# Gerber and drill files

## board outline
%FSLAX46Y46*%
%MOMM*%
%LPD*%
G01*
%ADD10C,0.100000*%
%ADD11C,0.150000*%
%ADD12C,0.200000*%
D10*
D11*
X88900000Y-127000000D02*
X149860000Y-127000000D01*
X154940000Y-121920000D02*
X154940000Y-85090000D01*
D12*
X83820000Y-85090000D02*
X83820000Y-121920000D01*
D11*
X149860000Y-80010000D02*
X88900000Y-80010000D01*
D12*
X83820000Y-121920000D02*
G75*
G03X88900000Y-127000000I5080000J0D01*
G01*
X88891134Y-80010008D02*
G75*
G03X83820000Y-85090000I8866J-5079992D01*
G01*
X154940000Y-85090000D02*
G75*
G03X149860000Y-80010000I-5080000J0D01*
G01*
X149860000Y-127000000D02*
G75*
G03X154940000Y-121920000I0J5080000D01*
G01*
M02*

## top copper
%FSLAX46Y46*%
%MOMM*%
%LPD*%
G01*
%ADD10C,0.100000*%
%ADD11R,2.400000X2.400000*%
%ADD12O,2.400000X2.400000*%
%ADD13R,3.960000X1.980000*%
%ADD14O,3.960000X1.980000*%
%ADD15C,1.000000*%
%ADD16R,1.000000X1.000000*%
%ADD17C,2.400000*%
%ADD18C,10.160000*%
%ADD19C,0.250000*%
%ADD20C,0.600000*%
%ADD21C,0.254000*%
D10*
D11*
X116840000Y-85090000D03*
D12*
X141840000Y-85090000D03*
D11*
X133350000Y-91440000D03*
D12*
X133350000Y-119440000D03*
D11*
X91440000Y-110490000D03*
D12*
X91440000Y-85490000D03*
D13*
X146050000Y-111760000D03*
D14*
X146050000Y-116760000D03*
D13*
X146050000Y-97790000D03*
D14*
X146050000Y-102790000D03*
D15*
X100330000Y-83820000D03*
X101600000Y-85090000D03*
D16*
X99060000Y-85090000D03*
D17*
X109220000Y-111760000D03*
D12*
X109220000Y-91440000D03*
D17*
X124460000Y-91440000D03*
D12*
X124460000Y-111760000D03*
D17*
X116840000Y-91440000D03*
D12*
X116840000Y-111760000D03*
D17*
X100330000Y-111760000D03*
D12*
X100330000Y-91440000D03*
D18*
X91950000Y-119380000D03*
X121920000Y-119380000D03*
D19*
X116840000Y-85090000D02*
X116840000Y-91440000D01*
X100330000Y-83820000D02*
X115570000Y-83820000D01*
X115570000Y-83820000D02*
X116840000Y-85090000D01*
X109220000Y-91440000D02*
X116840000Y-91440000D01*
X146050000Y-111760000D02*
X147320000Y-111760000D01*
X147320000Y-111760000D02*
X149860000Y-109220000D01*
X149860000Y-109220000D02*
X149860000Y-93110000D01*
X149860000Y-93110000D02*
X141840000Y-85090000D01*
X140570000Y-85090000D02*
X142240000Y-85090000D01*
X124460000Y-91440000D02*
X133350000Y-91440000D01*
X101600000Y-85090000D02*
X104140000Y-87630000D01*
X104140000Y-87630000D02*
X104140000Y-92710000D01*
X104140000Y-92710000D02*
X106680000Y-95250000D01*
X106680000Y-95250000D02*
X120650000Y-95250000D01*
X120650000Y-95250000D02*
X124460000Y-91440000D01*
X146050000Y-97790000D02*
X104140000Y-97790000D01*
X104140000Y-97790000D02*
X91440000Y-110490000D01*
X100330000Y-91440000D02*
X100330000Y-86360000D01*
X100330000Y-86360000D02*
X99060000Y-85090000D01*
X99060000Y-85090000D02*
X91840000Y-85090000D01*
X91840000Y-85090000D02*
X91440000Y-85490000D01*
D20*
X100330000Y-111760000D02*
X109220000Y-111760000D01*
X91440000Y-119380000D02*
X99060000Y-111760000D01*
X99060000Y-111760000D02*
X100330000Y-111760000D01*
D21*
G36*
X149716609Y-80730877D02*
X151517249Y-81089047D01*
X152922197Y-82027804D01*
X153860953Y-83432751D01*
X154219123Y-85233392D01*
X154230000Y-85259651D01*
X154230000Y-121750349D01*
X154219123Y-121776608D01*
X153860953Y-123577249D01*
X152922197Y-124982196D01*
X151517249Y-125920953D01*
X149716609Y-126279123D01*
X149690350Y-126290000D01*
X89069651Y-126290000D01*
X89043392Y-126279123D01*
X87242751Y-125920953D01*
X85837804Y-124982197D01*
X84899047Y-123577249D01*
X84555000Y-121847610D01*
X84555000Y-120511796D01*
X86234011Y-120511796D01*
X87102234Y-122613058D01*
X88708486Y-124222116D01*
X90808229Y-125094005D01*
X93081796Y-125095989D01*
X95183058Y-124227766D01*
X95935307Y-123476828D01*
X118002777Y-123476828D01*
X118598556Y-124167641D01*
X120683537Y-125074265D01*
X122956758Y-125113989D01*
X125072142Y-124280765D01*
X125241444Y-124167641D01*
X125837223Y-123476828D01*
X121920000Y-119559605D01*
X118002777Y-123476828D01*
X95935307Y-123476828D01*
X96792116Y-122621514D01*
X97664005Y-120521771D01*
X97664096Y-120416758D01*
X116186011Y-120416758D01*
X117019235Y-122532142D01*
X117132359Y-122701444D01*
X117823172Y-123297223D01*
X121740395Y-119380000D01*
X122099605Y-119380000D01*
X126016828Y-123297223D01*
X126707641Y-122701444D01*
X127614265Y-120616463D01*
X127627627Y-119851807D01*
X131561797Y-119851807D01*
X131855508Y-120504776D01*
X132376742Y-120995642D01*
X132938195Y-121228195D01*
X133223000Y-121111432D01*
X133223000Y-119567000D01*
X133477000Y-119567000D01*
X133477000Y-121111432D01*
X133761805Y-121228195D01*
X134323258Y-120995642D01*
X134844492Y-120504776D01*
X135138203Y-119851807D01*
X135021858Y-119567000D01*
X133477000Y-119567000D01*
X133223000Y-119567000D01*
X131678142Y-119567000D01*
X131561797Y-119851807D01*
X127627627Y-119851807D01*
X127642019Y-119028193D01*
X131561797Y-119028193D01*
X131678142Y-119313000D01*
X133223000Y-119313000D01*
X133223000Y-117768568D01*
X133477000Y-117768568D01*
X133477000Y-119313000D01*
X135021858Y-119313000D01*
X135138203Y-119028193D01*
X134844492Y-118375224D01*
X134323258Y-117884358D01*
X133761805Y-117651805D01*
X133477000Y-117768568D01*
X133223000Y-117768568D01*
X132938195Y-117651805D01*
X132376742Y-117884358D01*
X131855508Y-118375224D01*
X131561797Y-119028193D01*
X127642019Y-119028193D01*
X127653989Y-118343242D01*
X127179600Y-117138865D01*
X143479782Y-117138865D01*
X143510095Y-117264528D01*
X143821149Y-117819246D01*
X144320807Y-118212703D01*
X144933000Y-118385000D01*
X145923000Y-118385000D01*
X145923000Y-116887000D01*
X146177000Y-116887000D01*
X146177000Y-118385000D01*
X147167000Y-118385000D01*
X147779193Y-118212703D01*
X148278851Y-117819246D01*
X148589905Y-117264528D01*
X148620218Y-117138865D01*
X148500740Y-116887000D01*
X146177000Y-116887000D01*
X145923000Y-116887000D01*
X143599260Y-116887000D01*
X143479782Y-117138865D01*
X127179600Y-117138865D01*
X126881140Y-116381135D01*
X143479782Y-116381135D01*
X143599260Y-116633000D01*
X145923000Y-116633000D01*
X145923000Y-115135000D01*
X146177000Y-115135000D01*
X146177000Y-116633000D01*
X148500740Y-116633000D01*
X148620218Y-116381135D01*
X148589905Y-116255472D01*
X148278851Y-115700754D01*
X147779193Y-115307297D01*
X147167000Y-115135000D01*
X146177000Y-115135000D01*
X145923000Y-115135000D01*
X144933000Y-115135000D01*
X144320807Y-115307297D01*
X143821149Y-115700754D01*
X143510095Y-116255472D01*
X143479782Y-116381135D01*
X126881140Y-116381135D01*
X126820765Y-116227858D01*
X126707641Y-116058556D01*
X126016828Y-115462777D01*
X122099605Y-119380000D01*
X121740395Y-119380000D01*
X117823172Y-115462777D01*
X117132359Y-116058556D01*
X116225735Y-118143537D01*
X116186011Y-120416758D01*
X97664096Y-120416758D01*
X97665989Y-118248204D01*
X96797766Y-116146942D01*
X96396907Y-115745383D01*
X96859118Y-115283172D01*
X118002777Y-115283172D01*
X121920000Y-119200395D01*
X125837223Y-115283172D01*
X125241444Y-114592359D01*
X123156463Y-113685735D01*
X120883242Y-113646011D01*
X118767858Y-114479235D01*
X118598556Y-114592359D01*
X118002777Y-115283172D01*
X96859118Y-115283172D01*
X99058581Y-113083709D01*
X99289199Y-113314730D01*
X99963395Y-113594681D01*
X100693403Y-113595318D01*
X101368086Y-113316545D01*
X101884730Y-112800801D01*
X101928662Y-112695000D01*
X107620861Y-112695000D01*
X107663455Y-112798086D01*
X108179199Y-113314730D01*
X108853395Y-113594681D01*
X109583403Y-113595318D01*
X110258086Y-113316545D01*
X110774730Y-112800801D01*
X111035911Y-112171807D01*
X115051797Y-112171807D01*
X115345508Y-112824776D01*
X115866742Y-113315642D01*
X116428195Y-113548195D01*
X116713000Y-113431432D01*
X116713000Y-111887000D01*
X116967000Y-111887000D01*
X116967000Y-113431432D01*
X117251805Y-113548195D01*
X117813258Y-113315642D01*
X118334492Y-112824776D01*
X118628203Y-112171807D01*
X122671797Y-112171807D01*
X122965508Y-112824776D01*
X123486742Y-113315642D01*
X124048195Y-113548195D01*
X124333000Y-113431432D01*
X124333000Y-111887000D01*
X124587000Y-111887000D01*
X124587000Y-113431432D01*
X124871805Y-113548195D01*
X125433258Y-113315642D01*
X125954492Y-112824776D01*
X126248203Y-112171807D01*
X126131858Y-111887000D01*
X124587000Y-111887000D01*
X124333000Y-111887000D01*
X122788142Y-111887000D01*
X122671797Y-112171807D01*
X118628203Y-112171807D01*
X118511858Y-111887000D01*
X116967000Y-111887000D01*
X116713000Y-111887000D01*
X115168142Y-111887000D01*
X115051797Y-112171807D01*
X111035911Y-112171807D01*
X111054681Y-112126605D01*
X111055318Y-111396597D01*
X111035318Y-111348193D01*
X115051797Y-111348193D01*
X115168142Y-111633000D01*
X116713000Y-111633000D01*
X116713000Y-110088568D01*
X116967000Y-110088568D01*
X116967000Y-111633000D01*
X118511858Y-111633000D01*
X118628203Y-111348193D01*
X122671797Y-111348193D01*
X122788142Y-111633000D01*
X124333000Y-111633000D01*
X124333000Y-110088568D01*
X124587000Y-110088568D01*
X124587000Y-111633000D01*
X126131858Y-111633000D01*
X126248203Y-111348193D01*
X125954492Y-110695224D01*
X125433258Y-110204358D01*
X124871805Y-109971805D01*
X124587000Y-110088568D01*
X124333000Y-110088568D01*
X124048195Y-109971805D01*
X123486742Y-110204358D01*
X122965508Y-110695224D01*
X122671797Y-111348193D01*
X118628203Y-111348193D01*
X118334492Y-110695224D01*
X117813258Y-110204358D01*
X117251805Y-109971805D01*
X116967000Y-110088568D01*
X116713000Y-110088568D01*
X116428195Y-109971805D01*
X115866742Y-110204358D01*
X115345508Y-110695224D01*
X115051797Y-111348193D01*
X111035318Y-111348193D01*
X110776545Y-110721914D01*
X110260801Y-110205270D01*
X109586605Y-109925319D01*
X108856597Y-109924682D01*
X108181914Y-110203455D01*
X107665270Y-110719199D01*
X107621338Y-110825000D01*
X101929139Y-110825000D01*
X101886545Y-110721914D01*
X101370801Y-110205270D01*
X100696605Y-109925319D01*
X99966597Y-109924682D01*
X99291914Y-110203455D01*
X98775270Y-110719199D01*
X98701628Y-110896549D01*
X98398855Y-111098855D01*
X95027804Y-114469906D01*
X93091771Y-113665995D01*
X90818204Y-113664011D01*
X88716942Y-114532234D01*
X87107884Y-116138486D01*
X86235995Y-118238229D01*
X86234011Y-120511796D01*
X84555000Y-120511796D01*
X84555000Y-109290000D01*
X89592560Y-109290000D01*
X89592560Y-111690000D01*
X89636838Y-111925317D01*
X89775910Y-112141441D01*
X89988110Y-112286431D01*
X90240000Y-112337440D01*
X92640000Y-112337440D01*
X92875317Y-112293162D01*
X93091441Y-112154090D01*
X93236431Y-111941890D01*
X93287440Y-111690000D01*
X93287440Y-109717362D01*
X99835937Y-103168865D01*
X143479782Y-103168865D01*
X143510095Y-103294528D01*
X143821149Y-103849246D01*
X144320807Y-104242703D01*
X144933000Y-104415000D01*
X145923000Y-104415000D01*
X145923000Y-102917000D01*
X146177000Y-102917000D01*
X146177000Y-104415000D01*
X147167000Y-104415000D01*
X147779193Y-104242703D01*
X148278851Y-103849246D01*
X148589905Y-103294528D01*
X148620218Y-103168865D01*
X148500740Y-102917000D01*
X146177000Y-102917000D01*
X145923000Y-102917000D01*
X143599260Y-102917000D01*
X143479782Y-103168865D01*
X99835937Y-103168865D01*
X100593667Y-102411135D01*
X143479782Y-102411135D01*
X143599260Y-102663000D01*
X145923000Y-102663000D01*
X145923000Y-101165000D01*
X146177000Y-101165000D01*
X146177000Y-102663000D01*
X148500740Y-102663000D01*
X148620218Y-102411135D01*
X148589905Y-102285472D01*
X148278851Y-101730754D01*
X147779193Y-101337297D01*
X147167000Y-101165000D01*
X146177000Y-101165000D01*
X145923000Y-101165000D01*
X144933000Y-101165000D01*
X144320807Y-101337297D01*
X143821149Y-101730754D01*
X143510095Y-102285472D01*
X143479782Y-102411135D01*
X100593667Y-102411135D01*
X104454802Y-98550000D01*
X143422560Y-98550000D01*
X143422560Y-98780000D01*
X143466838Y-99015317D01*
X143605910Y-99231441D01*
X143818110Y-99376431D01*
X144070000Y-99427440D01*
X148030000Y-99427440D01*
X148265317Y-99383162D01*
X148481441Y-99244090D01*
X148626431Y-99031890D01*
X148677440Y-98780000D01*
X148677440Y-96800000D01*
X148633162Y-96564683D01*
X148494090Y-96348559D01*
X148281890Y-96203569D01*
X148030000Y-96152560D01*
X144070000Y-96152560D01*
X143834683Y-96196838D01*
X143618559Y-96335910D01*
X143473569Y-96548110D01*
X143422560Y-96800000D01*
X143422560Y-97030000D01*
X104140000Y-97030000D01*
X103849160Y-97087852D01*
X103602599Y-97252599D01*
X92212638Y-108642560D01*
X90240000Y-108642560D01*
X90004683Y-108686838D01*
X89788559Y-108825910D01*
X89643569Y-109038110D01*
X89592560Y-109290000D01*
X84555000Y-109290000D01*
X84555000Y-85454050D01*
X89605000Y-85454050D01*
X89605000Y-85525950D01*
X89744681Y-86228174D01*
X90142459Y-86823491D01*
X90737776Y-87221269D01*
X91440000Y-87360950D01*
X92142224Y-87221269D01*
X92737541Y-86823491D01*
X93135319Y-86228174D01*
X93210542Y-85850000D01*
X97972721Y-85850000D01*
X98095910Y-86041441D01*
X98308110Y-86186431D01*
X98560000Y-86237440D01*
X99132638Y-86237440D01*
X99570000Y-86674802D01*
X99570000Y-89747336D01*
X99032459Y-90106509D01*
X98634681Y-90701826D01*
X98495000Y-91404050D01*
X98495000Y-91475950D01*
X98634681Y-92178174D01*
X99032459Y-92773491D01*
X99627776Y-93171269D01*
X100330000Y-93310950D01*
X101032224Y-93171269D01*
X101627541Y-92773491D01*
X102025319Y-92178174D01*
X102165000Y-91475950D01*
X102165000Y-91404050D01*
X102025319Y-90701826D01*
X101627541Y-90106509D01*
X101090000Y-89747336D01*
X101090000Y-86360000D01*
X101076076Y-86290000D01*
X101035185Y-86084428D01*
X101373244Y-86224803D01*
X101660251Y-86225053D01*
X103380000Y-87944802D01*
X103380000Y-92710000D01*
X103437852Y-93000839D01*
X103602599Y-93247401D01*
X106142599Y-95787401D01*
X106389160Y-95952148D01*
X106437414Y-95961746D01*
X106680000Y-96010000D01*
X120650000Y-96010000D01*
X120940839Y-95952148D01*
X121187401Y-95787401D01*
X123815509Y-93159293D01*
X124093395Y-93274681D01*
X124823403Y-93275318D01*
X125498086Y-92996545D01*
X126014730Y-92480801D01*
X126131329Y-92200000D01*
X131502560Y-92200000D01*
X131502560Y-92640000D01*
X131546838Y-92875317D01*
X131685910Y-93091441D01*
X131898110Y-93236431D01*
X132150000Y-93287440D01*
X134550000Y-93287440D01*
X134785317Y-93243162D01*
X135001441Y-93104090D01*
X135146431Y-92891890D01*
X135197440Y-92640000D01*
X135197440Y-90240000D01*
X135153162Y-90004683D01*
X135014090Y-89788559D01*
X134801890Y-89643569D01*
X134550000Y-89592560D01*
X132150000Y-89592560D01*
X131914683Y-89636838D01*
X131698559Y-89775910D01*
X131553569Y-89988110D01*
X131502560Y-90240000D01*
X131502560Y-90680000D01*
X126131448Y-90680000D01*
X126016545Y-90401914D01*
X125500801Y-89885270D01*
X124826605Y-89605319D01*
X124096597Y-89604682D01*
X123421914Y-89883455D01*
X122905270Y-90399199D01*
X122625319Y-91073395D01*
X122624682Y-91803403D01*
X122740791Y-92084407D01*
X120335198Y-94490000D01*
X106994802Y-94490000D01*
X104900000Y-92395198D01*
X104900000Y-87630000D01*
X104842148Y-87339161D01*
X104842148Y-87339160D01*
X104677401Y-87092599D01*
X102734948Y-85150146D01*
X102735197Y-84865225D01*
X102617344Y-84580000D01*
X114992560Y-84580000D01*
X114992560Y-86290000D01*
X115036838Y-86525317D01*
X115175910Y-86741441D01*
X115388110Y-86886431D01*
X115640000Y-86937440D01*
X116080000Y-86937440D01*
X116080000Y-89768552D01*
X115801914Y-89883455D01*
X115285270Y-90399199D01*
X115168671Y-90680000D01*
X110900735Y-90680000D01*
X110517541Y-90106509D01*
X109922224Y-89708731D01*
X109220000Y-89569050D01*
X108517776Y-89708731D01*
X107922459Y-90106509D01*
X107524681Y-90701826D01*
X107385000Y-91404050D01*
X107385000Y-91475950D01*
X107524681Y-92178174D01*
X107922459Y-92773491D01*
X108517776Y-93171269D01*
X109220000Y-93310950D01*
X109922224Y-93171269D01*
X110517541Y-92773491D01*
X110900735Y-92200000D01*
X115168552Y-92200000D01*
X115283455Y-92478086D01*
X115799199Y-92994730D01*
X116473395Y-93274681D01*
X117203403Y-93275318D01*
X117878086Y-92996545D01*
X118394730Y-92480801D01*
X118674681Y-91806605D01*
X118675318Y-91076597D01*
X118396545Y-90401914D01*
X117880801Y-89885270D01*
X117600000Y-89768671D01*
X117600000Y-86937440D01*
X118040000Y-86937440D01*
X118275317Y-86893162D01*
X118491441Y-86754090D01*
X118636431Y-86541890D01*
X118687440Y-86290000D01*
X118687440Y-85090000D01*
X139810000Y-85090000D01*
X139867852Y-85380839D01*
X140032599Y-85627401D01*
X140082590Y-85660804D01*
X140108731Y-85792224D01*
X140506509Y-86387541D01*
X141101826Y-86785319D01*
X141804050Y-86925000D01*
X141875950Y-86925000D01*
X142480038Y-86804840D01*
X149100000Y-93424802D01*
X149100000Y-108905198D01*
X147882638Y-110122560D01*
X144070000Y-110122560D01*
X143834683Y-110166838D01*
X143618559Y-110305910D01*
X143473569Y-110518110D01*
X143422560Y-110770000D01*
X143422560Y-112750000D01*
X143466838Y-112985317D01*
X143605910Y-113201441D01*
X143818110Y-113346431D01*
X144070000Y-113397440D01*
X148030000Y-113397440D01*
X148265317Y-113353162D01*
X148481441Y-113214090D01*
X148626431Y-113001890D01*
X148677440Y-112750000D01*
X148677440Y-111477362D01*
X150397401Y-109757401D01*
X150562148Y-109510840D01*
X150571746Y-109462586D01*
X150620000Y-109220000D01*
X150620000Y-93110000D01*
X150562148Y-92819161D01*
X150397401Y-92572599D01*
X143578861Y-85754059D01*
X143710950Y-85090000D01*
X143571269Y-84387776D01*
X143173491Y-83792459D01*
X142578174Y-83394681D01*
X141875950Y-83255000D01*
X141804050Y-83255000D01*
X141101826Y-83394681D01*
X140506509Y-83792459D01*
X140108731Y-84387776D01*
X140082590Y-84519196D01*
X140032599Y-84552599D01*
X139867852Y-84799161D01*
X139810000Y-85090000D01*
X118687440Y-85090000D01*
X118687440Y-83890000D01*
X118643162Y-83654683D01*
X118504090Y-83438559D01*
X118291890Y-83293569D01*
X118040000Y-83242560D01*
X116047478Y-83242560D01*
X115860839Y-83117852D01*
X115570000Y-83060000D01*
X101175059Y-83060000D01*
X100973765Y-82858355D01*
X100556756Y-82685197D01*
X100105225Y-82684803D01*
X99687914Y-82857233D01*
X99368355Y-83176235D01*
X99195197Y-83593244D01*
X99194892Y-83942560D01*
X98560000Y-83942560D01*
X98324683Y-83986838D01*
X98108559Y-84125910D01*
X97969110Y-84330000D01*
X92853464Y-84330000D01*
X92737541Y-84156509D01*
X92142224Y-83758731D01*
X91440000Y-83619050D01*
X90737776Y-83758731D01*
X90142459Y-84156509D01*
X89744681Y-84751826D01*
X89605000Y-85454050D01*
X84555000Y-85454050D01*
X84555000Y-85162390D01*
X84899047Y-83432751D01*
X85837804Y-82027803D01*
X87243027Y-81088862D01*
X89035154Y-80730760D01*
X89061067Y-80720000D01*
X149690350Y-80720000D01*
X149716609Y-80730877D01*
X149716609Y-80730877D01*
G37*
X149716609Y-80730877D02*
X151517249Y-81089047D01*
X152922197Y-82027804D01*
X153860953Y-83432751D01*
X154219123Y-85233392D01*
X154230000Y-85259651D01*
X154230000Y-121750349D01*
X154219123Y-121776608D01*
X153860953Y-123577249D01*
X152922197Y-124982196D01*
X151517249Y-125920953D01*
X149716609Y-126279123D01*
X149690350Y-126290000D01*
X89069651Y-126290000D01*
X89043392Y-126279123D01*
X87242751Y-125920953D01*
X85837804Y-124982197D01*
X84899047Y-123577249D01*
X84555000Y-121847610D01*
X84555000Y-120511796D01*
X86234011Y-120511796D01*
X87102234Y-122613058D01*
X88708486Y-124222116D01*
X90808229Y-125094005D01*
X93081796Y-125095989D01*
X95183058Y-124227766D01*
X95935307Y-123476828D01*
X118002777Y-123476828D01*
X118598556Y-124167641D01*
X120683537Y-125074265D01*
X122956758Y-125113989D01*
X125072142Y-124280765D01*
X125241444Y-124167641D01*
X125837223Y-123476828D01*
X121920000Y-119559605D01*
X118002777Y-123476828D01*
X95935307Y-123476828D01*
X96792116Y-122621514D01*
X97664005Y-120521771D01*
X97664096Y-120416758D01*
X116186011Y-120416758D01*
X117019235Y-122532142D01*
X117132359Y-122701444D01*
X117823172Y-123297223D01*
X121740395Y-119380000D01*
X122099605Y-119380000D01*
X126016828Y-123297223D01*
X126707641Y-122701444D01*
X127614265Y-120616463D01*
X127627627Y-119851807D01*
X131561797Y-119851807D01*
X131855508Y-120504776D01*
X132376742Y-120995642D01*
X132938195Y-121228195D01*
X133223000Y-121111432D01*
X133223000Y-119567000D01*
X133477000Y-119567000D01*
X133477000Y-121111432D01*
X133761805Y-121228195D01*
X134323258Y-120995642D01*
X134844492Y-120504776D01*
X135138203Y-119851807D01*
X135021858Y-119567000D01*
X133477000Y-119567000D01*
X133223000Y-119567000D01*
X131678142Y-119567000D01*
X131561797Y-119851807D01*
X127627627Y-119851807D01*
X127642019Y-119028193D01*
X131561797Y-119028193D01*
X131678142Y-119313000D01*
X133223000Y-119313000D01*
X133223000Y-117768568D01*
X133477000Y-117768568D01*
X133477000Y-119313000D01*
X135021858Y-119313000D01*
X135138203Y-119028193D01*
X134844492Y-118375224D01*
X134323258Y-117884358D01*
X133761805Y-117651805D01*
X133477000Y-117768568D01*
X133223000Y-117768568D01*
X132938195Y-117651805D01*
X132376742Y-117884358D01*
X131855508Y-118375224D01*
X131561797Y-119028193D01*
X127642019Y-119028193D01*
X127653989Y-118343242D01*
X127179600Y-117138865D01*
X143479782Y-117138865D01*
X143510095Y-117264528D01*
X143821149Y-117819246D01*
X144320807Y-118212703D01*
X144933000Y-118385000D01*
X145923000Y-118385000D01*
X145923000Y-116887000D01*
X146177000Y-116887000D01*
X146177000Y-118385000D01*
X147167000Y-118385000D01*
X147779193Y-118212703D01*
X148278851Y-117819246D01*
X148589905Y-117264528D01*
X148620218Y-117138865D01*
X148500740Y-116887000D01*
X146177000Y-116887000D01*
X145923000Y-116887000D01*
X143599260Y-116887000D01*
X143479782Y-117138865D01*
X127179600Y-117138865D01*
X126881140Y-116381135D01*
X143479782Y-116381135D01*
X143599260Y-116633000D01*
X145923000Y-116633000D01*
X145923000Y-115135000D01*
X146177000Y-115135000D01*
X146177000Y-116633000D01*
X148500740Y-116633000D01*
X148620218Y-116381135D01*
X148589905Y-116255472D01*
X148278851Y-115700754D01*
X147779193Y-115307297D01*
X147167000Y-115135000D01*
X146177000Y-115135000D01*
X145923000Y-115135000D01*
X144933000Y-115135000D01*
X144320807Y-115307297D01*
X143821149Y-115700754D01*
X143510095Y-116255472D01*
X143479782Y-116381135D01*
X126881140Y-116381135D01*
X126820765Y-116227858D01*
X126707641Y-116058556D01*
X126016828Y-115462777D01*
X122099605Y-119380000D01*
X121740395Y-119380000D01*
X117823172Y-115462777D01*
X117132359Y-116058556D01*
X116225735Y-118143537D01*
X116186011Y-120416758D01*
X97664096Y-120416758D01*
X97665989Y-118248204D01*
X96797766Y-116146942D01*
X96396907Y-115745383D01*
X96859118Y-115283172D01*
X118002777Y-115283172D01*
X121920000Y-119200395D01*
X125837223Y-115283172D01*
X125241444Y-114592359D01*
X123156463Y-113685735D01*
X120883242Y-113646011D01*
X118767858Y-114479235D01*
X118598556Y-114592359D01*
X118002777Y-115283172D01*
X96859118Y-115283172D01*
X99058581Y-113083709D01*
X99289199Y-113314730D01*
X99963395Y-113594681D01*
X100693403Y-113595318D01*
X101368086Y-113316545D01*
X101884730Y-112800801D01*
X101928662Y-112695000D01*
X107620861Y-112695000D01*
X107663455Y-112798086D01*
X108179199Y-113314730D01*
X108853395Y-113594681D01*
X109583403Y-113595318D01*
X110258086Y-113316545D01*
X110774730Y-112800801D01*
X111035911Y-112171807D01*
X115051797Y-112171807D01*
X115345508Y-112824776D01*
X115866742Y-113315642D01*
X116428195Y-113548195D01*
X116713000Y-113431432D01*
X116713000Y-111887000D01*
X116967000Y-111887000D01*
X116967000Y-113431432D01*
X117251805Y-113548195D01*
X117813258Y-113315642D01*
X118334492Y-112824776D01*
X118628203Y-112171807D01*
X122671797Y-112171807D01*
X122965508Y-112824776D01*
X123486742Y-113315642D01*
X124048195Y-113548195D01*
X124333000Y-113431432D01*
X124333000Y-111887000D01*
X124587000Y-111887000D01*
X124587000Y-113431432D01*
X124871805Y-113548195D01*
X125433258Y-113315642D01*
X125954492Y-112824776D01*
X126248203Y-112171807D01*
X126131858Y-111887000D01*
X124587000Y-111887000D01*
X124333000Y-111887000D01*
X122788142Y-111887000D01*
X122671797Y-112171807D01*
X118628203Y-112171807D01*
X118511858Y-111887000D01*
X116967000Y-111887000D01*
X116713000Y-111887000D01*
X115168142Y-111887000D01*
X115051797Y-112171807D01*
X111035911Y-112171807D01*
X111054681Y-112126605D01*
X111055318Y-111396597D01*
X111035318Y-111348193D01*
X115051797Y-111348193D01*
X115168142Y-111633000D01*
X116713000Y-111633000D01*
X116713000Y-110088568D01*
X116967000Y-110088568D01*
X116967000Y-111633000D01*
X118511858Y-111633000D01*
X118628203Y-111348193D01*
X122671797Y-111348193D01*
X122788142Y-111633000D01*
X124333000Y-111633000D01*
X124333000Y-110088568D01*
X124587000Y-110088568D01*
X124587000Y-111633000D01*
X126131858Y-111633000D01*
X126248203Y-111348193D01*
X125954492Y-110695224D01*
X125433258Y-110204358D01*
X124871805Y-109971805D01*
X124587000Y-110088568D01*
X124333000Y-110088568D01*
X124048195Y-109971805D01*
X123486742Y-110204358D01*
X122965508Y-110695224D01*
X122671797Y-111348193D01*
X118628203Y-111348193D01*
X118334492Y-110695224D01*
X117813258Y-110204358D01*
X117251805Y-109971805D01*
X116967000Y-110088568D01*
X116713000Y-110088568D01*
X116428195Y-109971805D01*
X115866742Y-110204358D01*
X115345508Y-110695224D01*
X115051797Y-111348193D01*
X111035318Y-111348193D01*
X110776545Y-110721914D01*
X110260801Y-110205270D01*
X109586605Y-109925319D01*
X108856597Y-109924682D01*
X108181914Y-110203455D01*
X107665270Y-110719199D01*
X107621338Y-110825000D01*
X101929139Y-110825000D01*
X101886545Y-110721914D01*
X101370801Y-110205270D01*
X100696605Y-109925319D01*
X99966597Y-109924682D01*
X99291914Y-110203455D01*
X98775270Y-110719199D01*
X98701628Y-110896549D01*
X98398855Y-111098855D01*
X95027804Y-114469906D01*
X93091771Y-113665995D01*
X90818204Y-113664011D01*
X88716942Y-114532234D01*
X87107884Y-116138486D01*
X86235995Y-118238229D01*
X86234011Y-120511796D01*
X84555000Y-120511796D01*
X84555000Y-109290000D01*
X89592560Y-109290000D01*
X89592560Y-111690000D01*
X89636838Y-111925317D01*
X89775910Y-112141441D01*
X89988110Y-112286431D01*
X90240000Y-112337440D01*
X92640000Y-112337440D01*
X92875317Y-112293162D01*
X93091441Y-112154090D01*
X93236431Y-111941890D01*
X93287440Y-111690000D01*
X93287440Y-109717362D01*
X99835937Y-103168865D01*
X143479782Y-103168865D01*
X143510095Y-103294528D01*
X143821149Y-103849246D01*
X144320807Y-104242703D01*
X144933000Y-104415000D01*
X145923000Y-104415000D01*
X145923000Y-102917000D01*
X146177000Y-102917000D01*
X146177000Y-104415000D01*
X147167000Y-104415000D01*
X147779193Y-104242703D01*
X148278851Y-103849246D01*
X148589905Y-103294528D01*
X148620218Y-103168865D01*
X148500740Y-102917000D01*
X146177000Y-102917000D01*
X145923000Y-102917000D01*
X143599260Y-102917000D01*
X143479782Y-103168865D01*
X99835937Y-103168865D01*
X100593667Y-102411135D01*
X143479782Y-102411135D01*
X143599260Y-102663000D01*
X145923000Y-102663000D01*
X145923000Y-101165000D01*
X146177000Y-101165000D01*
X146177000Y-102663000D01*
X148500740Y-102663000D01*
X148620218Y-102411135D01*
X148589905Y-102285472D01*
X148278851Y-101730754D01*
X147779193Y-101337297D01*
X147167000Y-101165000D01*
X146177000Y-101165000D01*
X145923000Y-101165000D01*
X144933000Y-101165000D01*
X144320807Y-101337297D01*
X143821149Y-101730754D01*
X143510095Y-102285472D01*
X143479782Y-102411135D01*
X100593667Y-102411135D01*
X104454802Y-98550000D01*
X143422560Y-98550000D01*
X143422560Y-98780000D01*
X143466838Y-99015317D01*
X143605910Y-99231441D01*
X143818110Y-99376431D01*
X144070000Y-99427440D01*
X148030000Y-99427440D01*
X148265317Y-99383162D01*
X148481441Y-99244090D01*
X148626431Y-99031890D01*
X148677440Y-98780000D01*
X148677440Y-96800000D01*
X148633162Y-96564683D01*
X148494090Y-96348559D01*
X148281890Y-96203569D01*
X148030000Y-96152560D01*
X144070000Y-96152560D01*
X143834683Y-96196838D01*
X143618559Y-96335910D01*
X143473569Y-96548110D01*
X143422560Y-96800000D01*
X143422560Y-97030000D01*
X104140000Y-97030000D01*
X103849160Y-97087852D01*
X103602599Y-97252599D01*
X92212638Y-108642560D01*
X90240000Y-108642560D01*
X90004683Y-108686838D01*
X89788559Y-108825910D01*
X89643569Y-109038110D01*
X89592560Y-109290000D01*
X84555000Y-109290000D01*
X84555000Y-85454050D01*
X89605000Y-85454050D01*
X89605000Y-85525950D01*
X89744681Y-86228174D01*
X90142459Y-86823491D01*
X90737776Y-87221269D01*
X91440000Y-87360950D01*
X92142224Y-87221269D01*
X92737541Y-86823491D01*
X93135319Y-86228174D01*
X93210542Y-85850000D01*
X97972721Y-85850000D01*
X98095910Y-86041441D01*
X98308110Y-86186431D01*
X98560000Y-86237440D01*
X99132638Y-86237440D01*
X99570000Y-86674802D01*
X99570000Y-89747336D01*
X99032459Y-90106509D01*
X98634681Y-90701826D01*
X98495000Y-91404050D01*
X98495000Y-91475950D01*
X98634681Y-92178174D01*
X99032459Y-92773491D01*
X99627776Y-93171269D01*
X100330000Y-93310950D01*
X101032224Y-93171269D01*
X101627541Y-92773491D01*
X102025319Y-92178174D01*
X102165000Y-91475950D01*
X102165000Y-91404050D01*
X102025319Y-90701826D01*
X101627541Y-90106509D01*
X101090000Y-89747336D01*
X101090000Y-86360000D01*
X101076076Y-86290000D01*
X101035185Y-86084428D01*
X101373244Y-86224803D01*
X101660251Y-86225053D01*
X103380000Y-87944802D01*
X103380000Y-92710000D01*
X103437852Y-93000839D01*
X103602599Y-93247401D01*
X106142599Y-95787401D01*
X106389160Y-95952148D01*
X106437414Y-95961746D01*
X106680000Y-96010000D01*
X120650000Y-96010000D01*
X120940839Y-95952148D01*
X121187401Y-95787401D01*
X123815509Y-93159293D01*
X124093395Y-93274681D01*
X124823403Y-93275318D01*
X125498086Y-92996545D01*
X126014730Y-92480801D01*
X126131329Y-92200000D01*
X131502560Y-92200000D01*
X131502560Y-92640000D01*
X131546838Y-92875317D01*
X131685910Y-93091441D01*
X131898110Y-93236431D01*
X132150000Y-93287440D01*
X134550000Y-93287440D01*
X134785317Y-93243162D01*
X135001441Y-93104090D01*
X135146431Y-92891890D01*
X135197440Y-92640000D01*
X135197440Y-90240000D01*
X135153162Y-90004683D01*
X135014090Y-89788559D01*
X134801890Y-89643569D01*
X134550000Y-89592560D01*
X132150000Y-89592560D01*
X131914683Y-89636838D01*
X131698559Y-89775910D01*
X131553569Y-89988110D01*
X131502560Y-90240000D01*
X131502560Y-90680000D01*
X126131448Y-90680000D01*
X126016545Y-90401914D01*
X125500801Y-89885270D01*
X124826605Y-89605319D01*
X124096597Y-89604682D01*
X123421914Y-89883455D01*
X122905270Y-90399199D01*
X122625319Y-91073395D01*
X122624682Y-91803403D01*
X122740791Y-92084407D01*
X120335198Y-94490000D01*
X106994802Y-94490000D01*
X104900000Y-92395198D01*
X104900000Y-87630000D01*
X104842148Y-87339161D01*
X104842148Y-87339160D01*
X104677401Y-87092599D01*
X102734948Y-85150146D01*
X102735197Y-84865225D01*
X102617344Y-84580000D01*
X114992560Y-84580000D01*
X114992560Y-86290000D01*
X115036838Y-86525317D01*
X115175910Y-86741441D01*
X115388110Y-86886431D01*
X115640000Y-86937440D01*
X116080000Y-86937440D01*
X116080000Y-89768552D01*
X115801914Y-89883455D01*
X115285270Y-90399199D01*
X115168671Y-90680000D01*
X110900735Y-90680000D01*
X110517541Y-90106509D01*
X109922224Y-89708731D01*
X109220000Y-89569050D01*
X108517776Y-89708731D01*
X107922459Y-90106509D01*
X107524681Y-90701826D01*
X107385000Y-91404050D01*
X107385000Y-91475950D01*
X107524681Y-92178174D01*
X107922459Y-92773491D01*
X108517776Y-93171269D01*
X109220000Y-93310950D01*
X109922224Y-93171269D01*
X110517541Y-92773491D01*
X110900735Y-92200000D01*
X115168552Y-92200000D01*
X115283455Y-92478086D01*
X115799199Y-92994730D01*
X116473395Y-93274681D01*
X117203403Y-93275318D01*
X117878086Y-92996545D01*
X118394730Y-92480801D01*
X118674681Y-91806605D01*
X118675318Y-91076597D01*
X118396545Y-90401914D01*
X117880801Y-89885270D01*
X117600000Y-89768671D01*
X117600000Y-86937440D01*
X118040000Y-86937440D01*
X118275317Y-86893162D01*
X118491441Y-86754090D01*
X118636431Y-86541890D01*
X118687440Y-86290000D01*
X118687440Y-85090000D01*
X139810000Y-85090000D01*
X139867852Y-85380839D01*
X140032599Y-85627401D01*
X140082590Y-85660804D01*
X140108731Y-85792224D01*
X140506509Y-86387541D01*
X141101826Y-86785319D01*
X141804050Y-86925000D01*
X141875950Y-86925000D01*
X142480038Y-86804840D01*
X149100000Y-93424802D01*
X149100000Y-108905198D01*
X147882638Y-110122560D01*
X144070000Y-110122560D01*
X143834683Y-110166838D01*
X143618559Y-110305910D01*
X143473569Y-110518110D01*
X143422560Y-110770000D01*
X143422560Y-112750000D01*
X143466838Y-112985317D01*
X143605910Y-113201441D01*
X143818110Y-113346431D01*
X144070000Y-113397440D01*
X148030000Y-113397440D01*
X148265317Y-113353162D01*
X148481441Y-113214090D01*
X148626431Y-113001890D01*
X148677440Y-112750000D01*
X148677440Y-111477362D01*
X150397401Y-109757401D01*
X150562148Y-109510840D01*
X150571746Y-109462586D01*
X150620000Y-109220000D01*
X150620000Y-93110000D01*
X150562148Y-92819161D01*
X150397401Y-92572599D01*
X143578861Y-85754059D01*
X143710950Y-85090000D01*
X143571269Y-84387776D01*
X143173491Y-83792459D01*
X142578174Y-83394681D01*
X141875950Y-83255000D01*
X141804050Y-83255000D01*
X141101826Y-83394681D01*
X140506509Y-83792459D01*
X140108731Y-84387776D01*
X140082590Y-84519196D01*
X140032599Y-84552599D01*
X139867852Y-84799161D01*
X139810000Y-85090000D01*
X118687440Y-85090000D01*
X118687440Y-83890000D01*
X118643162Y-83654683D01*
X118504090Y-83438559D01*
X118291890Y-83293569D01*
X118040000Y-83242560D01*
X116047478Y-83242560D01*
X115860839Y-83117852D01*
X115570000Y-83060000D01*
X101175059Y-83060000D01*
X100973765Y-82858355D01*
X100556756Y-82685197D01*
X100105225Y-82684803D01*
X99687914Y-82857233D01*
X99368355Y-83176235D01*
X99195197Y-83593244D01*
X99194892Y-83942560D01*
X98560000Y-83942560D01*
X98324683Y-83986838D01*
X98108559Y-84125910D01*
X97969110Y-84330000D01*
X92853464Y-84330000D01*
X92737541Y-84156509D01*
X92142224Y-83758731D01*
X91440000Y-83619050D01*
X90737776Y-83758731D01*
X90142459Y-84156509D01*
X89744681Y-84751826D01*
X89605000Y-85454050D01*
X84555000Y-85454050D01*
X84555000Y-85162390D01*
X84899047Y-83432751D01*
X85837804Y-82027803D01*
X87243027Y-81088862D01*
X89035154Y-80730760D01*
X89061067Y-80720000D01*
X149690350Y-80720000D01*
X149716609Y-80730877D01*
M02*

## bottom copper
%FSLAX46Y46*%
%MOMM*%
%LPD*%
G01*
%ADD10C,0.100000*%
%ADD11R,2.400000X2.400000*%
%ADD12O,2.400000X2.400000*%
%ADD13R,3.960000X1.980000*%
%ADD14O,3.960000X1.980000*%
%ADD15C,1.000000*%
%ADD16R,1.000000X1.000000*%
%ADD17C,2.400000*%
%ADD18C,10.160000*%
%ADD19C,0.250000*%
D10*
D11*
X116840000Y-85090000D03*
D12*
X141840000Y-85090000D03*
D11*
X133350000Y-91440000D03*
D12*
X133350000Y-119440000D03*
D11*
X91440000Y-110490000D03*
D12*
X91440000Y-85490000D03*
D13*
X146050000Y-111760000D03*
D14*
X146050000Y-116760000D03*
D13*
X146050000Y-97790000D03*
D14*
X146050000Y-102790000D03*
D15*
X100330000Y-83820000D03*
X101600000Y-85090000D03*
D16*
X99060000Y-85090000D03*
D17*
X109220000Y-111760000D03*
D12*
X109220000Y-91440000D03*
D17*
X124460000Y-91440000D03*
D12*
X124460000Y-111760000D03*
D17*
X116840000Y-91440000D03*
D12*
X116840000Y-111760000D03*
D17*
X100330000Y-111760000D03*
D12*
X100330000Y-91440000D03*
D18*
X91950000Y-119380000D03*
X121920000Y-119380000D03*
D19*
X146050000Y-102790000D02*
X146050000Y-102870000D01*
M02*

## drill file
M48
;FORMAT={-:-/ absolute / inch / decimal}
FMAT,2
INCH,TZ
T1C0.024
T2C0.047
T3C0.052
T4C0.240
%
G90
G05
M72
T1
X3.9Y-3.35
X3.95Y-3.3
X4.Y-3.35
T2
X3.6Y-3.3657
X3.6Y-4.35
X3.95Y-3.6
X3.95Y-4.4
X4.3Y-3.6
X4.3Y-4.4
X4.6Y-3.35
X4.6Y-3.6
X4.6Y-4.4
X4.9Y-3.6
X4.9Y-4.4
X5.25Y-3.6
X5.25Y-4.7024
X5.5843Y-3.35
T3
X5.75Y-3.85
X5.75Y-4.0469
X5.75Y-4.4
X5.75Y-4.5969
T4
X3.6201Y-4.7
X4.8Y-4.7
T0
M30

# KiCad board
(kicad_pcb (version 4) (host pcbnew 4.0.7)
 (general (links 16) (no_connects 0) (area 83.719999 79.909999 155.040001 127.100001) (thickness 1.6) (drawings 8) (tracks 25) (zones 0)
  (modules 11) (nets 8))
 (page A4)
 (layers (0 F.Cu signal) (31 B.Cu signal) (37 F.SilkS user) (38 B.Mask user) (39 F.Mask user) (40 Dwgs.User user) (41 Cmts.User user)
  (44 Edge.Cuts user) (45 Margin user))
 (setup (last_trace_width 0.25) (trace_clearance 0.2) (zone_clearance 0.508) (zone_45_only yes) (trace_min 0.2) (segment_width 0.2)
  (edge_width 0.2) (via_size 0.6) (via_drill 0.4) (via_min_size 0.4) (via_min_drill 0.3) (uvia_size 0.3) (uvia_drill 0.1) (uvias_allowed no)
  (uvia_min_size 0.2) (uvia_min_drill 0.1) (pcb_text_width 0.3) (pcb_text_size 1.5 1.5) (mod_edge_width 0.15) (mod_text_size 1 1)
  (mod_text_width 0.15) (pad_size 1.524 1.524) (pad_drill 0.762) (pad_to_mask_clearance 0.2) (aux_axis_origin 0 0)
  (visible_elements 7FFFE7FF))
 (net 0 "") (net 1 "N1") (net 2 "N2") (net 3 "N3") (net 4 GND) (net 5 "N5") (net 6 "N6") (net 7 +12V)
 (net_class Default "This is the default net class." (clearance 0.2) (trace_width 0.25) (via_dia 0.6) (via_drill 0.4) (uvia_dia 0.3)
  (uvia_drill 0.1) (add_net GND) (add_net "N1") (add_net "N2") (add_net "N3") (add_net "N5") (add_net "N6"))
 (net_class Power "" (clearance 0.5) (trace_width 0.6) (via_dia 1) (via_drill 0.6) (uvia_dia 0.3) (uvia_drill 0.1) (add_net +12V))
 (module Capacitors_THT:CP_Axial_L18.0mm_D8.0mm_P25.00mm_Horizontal (layer F.Cu) (at 116.84 85.09)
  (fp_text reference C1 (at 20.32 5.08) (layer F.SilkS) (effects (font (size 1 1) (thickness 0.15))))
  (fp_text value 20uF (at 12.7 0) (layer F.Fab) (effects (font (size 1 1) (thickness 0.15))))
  (pad 1 thru_hole rect (at 0 0) (size 2.4 2.4) (drill 1.2) (layers *.Cu *.Mask) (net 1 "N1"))
  (pad 2 thru_hole oval (at 25 0) (size 2.4 2.4) (drill 1.2) (layers *.Cu *.Mask) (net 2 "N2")))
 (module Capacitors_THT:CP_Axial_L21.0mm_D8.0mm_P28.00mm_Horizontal (layer F.Cu) (at 133.35 91.44 270)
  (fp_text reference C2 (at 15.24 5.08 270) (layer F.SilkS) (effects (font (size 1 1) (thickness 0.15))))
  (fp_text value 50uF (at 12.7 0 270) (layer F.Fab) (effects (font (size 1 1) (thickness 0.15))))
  (pad 1 thru_hole rect (at 0 0 270) (size 2.4 2.4) (drill 1.2) (layers *.Cu *.Mask) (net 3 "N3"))
  (pad 2 thru_hole oval (at 28 0 270) (size 2.4 2.4) (drill 1.2) (layers *.Cu *.Mask) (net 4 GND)))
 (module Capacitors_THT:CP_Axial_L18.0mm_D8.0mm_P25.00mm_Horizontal (layer F.Cu) (at 91.44 110.49 90)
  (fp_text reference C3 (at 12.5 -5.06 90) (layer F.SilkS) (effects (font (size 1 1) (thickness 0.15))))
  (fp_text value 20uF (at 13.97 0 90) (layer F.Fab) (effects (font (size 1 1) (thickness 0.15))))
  (pad 1 thru_hole rect (at 0 0 90) (size 2.4 2.4) (drill 1.2) (layers *.Cu *.Mask) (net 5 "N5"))
  (pad 2 thru_hole oval (at 25 0 90) (size 2.4 2.4) (drill 1.2) (layers *.Cu *.Mask) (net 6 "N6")))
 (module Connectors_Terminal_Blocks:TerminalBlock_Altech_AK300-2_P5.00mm (layer F.Cu) (at 146.05 111.76 270)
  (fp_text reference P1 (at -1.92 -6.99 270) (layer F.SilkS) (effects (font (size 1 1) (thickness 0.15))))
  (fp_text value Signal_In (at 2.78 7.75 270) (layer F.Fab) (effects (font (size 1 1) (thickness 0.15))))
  (pad 1 thru_hole rect (at 0 0 270) (size 1.98 3.96) (drill 1.32) (layers *.Cu *.Mask) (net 2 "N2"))
  (pad 2 thru_hole oval (at 5 0 270) (size 1.98 3.96) (drill 1.32) (layers *.Cu *.Mask) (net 4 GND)))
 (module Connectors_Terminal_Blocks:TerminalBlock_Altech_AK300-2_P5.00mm (layer F.Cu) (at 146.05 97.79 270)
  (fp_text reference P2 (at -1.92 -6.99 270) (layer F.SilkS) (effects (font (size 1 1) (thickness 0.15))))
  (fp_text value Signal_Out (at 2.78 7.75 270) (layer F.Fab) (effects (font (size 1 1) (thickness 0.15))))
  (pad 1 thru_hole rect (at 0 0 270) (size 1.98 3.96) (drill 1.32) (layers *.Cu *.Mask) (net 5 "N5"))
  (pad 2 thru_hole oval (at 5 0 270) (size 1.98 3.96) (drill 1.32) (layers *.Cu *.Mask) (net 4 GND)))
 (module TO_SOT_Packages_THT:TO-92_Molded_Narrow (layer F.Cu) (at 99.06 85.09)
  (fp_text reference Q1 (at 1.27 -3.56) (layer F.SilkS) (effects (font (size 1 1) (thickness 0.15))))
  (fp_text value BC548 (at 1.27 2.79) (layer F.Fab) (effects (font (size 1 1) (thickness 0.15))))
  (pad 2 thru_hole circle (at 1.27 -1.27 90) (size 1 1) (drill 0.6) (layers *.Cu *.Mask) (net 1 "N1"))
  (pad 3 thru_hole circle (at 2.54 0 90) (size 1 1) (drill 0.6) (layers *.Cu *.Mask) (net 3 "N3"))
  (pad 1 thru_hole rect (at 0 0 90) (size 1 1) (drill 0.6) (layers *.Cu *.Mask) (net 6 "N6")))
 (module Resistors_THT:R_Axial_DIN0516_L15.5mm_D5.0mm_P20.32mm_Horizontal (layer F.Cu) (at 109.22 111.76 90)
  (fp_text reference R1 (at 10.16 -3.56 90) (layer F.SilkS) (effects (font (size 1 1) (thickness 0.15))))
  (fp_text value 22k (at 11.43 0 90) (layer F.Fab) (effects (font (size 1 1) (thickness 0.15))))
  (pad 1 thru_hole circle (at 0 0 90) (size 2.4 2.4) (drill 1.2) (layers *.Cu *.Mask) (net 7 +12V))
  (pad 2 thru_hole oval (at 20.32 0 90) (size 2.4 2.4) (drill 1.2) (layers *.Cu *.Mask) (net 1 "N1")))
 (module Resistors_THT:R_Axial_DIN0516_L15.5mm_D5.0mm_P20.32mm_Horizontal (layer F.Cu) (at 124.46 91.44 270)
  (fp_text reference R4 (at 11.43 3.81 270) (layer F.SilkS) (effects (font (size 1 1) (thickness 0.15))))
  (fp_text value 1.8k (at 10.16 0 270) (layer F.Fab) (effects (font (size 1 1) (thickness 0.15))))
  (pad 1 thru_hole circle (at 0 0 270) (size 2.4 2.4) (drill 1.2) (layers *.Cu *.Mask) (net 3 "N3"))
  (pad 2 thru_hole oval (at 20.32 0 270) (size 2.4 2.4) (drill 1.2) (layers *.Cu *.Mask) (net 4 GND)))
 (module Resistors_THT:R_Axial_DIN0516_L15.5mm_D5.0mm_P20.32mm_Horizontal (layer F.Cu) (at 116.84 91.44 270)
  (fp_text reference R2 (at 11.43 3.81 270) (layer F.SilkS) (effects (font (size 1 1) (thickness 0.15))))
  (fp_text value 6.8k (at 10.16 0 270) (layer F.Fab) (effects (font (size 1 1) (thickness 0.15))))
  (pad 1 thru_hole circle (at 0 0 270) (size 2.4 2.4) (drill 1.2) (layers *.Cu *.Mask) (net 1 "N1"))
  (pad 2 thru_hole oval (at 20.32 0 270) (size 2.4 2.4) (drill 1.2) (layers *.Cu *.Mask) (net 4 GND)))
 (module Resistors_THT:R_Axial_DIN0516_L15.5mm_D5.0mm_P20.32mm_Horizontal (layer F.Cu) (at 100.33 111.76 90)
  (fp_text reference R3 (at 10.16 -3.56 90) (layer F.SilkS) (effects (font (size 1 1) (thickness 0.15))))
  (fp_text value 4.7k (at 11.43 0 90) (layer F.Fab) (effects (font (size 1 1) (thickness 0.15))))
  (pad 1 thru_hole circle (at 0 0 90) (size 2.4 2.4) (drill 1.2) (layers *.Cu *.Mask) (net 7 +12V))
  (pad 2 thru_hole oval (at 20.32 0 90) (size 2.4 2.4) (drill 1.2) (layers *.Cu *.Mask) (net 6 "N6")))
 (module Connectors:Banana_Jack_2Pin (layer F.Cu) (at 91.95 119.38)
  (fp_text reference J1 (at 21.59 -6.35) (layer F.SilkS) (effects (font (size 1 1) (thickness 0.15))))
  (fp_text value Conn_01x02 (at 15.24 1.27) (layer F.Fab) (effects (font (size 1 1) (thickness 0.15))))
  (pad 1 thru_hole circle (at 0 0) (size 10.16 10.16) (drill 6.1) (layers *.Cu *.Mask) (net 7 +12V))
  (pad 2 thru_hole circle (at 29.97 0) (size 10.16 10.16) (drill 6.1) (layers *.Cu *.Mask) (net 4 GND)))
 (gr_line (start 88.9 127) (end 149.86 127) (angle 90) (layer Edge.Cuts) (width 0.15))
 (gr_line (start 154.94 121.92) (end 154.94 85.09) (angle 90) (layer Edge.Cuts) (width 0.15))
 (gr_line (start 83.82 85.09) (end 83.82 121.92) (layer Edge.Cuts) (width 0.2))
 (gr_line (start 149.86 80.01) (end 88.9 80.01) (angle 90) (layer Edge.Cuts) (width 0.15))
 (gr_arc (start 88.9 121.92) (end 88.9 127) (angle 90) (layer Edge.Cuts) (width 0.2))
 (gr_arc (start 88.9 85.09) (end 83.82 85.09) (angle 89.9) (layer Edge.Cuts) (width 0.2))
 (gr_arc (start 149.86 85.09) (end 149.86 80.01) (angle 90) (layer Edge.Cuts) (width 0.2))
 (gr_arc (start 149.86 121.92) (end 154.94 121.92) (angle 90) (layer Edge.Cuts) (width 0.2))
 (segment (start 116.84 85.09) (end 116.84 91.44) (width 0.25) (layer F.Cu) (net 1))
 (segment (start 100.33 83.82) (end 115.57 83.82) (width 0.25) (layer F.Cu) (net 1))
 (segment (start 115.57 83.82) (end 116.84 85.09) (width 0.25) (layer F.Cu) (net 1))
 (segment (start 109.22 91.44) (end 116.84 91.44) (width 0.25) (layer F.Cu) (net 1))
 (segment (start 146.05 111.76) (end 147.32 111.76) (width 0.25) (layer F.Cu) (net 2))
 (segment (start 147.32 111.76) (end 149.86 109.22) (width 0.25) (layer F.Cu) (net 2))
 (segment (start 149.86 109.22) (end 149.86 93.11) (width 0.25) (layer F.Cu) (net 2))
 (segment (start 149.86 93.11) (end 141.84 85.09) (width 0.25) (layer F.Cu) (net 2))
 (segment (start 140.57 85.09) (end 142.24 85.09) (width 0.25) (layer F.Cu) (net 2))
 (segment (start 124.46 91.44) (end 133.35 91.44) (width 0.25) (layer F.Cu) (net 3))
 (segment (start 101.6 85.09) (end 104.14 87.63) (width 0.25) (layer F.Cu) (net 3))
 (segment (start 104.14 87.63) (end 104.14 92.71) (width 0.25) (layer F.Cu) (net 3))
 (segment (start 104.14 92.71) (end 106.68 95.25) (width 0.25) (layer F.Cu) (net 3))
 (segment (start 106.68 95.25) (end 120.65 95.25) (width 0.25) (layer F.Cu) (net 3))
 (segment (start 120.65 95.25) (end 124.46 91.44) (width 0.25) (layer F.Cu) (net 3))
 (segment (start 146.05 102.79) (end 146.05 102.87) (width 0.25) (layer B.Cu) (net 4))
 (segment (start 146.05 97.79) (end 104.14 97.79) (width 0.25) (layer F.Cu) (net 5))
 (segment (start 104.14 97.79) (end 91.44 110.49) (width 0.25) (layer F.Cu) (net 5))
 (segment (start 100.33 91.44) (end 100.33 86.36) (width 0.25) (layer F.Cu) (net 6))
 (segment (start 100.33 86.36) (end 99.06 85.09) (width 0.25) (layer F.Cu) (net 6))
 (segment (start 99.06 85.09) (end 91.84 85.09) (width 0.25) (layer F.Cu) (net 6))
 (segment (start 91.84 85.09) (end 91.44 85.49) (width 0.25) (layer F.Cu) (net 6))
 (segment (start 100.33 111.76) (end 109.22 111.76) (width 0.6) (layer F.Cu) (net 7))
 (segment (start 91.44 119.38) (end 99.06 111.76) (width 0.6) (layer F.Cu) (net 7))
 (segment (start 99.06 111.76) (end 100.33 111.76) (width 0.6) (layer F.Cu) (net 7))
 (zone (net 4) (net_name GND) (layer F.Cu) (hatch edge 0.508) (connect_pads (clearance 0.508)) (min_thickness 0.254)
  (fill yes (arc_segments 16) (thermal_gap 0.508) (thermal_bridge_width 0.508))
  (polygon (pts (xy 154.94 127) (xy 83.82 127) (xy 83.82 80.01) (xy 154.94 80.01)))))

